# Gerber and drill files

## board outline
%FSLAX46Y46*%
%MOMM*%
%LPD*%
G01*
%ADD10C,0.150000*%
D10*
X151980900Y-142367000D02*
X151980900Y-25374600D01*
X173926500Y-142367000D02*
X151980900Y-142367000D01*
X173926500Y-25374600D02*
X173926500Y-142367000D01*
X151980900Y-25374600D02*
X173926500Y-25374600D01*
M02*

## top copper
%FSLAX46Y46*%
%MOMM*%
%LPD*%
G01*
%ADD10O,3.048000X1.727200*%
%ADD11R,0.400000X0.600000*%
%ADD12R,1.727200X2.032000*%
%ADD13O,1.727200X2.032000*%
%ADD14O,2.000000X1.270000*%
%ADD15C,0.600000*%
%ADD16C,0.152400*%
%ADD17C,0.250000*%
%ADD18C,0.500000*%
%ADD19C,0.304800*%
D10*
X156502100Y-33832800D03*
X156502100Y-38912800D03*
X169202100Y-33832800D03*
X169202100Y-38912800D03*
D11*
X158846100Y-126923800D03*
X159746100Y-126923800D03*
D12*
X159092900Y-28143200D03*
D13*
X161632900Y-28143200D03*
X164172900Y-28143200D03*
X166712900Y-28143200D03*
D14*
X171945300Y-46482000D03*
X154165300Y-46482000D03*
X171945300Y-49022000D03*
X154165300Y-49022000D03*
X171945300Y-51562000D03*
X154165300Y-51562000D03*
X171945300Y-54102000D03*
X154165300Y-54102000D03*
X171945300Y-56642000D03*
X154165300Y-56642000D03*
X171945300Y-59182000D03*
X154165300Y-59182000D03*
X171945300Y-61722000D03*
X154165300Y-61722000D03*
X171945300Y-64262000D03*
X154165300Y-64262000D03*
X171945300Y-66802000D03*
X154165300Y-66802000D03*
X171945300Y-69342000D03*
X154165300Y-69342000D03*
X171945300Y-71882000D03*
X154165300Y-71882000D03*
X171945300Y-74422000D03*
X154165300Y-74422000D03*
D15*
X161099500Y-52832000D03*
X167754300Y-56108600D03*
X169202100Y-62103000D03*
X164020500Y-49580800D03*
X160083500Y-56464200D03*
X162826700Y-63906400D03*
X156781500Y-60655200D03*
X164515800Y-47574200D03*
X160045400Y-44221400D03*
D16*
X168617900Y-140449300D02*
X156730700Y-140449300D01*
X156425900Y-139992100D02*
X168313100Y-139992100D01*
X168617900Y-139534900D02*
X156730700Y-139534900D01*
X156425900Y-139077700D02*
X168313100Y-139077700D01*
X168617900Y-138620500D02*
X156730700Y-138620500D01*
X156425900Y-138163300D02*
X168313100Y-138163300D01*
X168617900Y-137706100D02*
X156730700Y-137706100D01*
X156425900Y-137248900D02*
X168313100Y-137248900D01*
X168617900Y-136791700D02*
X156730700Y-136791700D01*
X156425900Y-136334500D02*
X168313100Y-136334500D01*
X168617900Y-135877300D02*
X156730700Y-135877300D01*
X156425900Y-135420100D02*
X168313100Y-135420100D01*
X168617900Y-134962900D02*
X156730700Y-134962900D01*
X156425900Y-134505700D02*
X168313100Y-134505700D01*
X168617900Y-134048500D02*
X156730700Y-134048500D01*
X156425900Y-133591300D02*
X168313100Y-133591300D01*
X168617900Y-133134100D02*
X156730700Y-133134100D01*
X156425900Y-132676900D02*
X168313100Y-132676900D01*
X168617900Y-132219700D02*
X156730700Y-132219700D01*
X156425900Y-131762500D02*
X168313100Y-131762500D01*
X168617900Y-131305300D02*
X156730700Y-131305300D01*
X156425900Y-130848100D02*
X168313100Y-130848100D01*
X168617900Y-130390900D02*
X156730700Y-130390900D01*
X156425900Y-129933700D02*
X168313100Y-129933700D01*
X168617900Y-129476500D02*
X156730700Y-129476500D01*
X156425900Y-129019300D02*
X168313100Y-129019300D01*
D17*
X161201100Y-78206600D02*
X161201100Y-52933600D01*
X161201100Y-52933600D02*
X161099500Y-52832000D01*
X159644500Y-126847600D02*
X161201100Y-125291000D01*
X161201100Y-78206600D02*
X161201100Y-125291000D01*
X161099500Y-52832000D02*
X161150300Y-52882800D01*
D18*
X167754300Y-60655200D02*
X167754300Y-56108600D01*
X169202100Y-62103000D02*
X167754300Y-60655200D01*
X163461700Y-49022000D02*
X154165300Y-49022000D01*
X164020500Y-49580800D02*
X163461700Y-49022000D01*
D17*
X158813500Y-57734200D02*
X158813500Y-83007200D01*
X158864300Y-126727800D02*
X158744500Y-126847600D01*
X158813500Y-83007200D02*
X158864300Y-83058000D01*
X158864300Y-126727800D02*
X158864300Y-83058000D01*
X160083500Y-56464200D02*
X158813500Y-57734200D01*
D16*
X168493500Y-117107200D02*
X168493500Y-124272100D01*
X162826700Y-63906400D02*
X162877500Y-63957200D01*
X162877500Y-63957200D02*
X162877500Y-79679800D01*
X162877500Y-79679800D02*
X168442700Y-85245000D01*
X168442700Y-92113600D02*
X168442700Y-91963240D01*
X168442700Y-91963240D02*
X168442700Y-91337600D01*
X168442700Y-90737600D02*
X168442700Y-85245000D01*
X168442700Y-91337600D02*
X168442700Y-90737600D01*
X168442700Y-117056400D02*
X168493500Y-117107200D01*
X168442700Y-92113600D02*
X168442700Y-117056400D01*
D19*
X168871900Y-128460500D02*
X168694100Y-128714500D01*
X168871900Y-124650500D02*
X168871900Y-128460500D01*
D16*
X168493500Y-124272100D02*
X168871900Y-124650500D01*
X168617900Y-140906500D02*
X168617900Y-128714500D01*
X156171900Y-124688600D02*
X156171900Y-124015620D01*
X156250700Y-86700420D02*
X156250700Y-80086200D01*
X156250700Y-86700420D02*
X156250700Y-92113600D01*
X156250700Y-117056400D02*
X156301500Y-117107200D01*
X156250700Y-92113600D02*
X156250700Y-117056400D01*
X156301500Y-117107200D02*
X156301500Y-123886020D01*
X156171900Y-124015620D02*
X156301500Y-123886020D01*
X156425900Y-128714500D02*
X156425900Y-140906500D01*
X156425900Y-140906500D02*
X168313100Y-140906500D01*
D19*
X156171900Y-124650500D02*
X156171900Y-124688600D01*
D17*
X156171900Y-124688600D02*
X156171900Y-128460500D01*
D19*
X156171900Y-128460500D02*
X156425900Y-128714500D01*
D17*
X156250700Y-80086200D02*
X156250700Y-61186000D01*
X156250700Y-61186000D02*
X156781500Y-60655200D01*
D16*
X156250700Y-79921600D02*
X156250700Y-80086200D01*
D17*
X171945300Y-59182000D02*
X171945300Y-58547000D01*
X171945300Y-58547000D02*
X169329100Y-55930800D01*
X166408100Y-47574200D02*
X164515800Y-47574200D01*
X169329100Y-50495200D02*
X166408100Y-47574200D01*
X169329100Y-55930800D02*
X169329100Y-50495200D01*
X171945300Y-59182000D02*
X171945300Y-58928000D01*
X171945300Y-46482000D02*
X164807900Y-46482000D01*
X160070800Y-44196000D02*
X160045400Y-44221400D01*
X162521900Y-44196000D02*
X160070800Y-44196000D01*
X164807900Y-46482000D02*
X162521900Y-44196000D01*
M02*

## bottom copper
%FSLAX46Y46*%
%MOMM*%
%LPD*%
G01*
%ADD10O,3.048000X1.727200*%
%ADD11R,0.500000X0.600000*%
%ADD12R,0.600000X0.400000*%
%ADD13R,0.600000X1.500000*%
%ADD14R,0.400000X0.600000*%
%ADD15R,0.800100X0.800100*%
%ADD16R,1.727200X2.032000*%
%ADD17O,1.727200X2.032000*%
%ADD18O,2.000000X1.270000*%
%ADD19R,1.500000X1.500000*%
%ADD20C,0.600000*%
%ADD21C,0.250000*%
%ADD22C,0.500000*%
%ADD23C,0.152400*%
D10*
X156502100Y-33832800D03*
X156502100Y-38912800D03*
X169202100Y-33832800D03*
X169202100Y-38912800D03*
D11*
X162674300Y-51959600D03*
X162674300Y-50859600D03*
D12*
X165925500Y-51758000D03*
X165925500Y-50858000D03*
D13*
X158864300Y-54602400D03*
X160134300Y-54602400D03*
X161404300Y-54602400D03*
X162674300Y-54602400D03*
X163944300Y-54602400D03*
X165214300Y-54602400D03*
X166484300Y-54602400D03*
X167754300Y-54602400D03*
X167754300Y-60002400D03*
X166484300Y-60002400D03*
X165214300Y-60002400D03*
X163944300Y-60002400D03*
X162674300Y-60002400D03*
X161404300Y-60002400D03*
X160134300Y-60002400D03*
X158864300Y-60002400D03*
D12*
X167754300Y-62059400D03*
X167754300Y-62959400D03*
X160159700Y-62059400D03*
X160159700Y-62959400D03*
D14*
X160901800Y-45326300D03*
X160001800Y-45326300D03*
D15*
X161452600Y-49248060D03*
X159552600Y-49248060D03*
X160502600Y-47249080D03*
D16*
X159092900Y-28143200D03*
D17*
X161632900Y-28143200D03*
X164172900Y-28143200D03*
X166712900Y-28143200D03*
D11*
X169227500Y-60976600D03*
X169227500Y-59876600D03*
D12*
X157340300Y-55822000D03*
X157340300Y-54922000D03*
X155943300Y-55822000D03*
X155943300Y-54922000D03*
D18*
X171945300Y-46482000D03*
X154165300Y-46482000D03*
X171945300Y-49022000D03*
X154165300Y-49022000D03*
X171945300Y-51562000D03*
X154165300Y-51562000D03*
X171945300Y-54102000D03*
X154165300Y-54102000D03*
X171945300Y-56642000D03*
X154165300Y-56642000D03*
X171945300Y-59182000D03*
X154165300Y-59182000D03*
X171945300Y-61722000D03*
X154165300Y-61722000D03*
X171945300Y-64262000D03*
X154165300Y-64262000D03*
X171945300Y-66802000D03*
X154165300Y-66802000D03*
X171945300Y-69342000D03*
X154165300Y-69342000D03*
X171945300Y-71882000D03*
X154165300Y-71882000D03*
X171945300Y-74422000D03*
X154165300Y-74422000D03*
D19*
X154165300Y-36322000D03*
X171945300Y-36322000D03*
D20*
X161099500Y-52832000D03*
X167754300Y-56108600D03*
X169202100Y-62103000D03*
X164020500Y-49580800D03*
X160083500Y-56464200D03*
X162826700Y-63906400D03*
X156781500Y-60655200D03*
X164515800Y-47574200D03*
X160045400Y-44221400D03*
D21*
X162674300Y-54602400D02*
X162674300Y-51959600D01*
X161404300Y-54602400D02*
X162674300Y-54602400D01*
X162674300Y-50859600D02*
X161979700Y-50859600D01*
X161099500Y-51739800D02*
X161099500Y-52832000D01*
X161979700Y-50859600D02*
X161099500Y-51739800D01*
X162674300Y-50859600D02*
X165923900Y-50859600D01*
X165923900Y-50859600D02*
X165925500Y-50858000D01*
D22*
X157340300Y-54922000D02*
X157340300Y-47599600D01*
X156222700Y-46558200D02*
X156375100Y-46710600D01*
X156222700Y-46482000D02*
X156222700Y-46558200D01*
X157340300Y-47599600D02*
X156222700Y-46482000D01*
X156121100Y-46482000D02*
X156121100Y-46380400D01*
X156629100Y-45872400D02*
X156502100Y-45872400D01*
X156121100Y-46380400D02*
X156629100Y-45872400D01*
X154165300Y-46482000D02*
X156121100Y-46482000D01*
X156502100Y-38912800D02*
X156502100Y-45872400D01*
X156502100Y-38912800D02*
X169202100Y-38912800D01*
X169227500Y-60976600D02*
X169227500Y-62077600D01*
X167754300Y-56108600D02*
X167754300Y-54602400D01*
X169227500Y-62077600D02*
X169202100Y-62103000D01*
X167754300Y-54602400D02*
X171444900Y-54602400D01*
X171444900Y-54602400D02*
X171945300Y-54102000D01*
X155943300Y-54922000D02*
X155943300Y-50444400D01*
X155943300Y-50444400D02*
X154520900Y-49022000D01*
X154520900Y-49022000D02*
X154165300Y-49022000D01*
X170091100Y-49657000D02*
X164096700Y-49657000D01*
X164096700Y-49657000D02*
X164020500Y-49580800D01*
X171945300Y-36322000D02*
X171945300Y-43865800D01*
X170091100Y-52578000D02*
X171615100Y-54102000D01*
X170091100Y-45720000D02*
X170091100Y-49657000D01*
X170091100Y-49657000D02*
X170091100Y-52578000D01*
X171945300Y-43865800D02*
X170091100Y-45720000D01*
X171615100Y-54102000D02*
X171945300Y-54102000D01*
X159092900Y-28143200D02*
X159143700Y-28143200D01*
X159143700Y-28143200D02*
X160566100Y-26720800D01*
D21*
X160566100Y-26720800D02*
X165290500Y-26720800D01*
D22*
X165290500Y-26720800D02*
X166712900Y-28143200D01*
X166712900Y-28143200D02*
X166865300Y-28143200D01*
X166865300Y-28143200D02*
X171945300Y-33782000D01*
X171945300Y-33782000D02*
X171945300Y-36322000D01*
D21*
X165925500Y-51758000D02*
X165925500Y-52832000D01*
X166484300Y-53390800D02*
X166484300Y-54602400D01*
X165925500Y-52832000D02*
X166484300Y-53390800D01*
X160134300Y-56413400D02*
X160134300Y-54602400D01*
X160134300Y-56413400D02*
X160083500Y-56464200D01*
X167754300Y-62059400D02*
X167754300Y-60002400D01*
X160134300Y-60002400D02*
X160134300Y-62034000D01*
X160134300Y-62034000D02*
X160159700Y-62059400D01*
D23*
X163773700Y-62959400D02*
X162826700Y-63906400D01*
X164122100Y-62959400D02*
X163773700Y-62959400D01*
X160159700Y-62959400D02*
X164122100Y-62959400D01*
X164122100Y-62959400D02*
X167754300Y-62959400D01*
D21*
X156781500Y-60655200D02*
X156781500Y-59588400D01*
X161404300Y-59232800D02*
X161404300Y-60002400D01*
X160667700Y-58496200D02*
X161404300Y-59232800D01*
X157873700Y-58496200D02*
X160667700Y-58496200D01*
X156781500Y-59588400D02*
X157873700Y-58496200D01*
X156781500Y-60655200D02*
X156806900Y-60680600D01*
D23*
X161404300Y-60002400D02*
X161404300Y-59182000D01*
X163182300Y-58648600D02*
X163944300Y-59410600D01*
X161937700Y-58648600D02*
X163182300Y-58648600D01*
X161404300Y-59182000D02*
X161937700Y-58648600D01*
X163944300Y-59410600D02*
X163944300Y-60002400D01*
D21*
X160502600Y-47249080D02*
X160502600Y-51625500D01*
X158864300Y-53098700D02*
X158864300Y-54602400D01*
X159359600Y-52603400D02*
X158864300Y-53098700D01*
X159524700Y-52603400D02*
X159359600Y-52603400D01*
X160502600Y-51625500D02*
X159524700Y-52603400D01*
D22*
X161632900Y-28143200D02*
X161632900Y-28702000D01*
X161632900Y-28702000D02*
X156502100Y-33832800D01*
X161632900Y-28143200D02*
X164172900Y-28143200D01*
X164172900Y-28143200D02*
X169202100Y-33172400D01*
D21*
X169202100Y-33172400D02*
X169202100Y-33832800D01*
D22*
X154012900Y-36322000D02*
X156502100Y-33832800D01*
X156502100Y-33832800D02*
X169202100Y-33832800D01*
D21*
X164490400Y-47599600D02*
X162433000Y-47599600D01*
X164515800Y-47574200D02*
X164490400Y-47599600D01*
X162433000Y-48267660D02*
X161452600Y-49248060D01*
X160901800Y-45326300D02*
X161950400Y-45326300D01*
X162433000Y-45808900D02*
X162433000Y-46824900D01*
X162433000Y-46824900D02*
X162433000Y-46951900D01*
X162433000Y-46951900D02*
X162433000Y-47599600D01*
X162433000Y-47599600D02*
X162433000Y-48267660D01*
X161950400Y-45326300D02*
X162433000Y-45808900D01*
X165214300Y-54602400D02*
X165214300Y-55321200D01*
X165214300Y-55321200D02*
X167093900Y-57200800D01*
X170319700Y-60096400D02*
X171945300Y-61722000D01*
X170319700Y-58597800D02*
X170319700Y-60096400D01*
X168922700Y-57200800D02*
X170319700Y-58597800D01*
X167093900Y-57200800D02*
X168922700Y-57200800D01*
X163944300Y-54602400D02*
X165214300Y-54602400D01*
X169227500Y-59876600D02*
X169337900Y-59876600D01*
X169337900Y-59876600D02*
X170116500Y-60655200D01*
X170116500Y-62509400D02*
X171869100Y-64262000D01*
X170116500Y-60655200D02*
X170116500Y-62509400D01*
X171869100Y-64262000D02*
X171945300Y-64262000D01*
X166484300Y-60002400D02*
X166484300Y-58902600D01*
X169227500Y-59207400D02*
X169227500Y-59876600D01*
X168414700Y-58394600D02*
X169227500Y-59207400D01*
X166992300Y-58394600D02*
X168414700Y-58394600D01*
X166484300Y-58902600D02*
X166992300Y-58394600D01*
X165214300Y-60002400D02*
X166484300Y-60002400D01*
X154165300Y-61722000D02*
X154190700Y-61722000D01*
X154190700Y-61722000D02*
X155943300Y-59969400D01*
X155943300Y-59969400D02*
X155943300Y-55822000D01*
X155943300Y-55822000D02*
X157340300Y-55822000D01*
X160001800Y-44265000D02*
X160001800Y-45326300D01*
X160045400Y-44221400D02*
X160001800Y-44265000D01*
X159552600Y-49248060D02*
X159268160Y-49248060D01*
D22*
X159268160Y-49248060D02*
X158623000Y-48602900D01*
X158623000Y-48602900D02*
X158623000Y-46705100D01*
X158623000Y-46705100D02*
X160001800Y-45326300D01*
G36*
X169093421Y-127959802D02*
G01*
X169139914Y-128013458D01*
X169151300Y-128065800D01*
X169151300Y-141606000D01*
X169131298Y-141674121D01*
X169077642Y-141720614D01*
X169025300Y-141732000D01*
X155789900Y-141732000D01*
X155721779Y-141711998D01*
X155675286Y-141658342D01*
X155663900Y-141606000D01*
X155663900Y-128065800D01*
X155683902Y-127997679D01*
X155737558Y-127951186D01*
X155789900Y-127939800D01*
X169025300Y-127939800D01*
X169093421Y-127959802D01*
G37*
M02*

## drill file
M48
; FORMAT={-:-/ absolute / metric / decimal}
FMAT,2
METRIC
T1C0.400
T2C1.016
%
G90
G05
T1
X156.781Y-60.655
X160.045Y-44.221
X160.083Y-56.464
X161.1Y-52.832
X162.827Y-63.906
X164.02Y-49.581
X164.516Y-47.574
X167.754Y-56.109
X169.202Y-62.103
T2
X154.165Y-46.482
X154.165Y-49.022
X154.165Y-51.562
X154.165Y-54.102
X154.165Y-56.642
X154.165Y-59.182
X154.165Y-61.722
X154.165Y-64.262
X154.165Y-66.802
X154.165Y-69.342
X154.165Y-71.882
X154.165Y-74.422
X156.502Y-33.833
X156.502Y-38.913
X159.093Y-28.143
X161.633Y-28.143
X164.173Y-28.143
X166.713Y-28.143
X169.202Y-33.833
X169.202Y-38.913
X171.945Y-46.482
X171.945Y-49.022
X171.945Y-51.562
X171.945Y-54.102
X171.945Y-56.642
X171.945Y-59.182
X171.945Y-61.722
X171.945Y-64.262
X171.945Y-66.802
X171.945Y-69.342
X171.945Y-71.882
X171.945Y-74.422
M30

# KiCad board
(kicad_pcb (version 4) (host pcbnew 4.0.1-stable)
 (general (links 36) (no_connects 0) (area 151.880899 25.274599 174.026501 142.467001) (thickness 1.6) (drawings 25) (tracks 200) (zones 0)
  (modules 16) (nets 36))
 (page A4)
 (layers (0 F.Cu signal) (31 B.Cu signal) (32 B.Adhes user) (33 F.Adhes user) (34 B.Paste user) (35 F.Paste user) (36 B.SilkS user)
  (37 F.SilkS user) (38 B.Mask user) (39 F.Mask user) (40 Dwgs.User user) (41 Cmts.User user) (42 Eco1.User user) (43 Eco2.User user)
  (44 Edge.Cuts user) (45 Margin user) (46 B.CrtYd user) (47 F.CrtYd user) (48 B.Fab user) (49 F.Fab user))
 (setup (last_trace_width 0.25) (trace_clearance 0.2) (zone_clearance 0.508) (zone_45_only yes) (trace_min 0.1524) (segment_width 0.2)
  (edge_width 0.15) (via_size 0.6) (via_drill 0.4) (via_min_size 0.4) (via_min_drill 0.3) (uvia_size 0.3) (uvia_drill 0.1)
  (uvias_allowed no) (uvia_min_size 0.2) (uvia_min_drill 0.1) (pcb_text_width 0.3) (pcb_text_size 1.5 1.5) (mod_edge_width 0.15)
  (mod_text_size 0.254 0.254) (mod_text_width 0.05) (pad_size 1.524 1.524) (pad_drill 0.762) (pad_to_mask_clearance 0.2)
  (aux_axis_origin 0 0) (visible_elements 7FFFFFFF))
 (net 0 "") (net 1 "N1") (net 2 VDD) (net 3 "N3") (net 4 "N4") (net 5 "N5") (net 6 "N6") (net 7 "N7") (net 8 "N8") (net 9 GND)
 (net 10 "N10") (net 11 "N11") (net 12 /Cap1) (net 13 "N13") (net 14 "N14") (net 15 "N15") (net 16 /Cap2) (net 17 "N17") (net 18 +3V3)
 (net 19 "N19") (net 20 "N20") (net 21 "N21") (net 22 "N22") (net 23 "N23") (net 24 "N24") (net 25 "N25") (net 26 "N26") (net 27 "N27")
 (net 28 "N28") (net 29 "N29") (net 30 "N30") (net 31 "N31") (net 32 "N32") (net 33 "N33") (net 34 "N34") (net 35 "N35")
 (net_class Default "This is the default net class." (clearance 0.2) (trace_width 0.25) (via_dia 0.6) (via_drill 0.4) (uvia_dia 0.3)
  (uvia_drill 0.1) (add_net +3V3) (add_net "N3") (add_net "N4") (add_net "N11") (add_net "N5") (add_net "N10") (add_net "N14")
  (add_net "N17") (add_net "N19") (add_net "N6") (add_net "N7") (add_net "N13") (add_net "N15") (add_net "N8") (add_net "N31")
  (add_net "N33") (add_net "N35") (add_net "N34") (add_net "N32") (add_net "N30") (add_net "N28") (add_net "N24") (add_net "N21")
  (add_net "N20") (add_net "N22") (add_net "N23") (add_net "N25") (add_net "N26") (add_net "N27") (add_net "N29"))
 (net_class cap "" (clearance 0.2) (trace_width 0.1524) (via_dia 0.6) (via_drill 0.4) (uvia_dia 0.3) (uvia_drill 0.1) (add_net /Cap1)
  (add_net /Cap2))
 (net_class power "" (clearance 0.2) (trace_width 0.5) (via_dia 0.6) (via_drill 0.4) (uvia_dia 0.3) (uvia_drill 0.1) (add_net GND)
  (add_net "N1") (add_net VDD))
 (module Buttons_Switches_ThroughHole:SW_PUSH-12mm (layer B.Cu) (at 162.8521 36.3728 180)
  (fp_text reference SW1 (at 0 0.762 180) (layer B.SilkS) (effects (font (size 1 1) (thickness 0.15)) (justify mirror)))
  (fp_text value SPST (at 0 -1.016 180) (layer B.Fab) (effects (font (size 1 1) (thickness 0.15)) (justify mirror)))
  (pad 1 thru_hole oval (at 6.35 2.54 180) (size 3.048 1.7272) (drill 1.016) (layers *.Cu *.Mask B.SilkS) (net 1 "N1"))
  (pad 2 thru_hole oval (at 6.35 -2.54 180) (size 3.048 1.7272) (drill 1.016) (layers *.Cu *.Mask B.SilkS) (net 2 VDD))
  (pad 1 thru_hole oval (at -6.35 2.54 180) (size 3.048 1.7272) (drill 1.016) (layers *.Cu *.Mask B.SilkS) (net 1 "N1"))
  (pad 2 thru_hole oval (at -6.35 -2.54 180) (size 3.048 1.7272) (drill 1.016) (layers *.Cu *.Mask B.SilkS) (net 2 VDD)))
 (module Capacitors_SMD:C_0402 (layer B.Cu) (at 162.6743 51.4096 90)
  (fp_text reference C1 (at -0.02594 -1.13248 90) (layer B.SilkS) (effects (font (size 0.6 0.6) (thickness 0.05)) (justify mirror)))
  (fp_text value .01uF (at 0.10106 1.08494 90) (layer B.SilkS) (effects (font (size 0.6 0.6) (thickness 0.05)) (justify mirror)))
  (pad 1 smd rect (at -0.55 0 90) (size 0.6 0.5) (layers B.Cu B.Paste B.Mask) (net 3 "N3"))
  (pad 2 smd rect (at 0.55 0 90) (size 0.6 0.5) (layers B.Cu B.Paste B.Mask) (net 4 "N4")))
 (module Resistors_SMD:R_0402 (layer B.Cu) (at 165.9255 51.308 90)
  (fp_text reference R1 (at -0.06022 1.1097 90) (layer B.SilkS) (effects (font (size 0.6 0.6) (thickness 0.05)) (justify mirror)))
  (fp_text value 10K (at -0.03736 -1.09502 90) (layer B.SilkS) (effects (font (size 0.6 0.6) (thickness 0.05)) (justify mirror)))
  (pad 1 smd rect (at -0.45 0 90) (size 0.4 0.6) (layers B.Cu B.Paste B.Mask) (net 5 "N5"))
  (pad 2 smd rect (at 0.45 0 90) (size 0.4 0.6) (layers B.Cu B.Paste B.Mask) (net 4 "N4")))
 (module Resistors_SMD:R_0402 (layer F.Cu) (at 159.2961 126.9238)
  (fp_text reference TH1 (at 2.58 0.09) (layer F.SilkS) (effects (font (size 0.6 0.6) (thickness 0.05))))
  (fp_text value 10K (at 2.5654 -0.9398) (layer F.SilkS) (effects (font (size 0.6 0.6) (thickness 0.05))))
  (pad 1 smd rect (at -0.45 0) (size 0.4 0.6) (layers F.Cu F.Paste F.Mask) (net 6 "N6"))
  (pad 2 smd rect (at 0.45 0) (size 0.4 0.6) (layers F.Cu F.Paste F.Mask) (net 4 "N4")))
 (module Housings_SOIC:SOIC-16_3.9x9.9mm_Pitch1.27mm (layer B.Cu) (at 163.3093 57.3024 270)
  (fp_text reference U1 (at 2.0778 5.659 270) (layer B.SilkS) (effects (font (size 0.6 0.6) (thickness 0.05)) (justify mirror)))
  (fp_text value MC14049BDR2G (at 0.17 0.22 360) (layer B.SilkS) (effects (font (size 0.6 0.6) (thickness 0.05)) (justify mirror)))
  (pad 1 smd rect (at -2.7 4.445 270) (size 1.5 0.6) (layers B.Cu B.Paste B.Mask) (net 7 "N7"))
  (pad 2 smd rect (at -2.7 3.175 270) (size 1.5 0.6) (layers B.Cu B.Paste B.Mask) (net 6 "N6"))
  (pad 3 smd rect (at -2.7 1.905 270) (size 1.5 0.6) (layers B.Cu B.Paste B.Mask) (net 3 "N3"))
  (pad 4 smd rect (at -2.7 0.635 270) (size 1.5 0.6) (layers B.Cu B.Paste B.Mask) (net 3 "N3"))
  (pad 5 smd rect (at -2.7 -0.635 270) (size 1.5 0.6) (layers B.Cu B.Paste B.Mask) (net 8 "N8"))
  (pad 6 smd rect (at -2.7 -1.905 270) (size 1.5 0.6) (layers B.Cu B.Paste B.Mask) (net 8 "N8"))
  (pad 7 smd rect (at -2.7 -3.175 270) (size 1.5 0.6) (layers B.Cu B.Paste B.Mask) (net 5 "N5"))
  (pad 8 smd rect (at -2.7 -4.445 270) (size 1.5 0.6) (layers B.Cu B.Paste B.Mask) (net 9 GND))
  (pad 9 smd rect (at 2.7 -4.445 270) (size 1.5 0.6) (layers B.Cu B.Paste B.Mask) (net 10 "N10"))
  (pad 10 smd rect (at 2.7 -3.175 270) (size 1.5 0.6) (layers B.Cu B.Paste B.Mask) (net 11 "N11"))
  (pad 11 smd rect (at 2.7 -1.905 270) (size 1.5 0.6) (layers B.Cu B.Paste B.Mask) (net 11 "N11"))
  (pad 12 smd rect (at 2.7 -0.635 270) (size 1.5 0.6) (layers B.Cu B.Paste B.Mask) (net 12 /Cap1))
  (pad 13 smd rect (at 2.7 0.635 270) (size 1.5 0.6) (layers B.Cu B.Paste B.Mask) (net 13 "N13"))
  (pad 14 smd rect (at 2.7 1.905 270) (size 1.5 0.6) (layers B.Cu B.Paste B.Mask) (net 12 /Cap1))
  (pad 15 smd rect (at 2.7 3.175 270) (size 1.5 0.6) (layers B.Cu B.Paste B.Mask) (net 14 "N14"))
  (pad 16 smd rect (at 2.7 4.445 270) (size 1.5 0.6) (layers B.Cu B.Paste B.Mask) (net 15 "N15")))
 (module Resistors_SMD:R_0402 (layer B.Cu) (at 167.7543 62.5094 270)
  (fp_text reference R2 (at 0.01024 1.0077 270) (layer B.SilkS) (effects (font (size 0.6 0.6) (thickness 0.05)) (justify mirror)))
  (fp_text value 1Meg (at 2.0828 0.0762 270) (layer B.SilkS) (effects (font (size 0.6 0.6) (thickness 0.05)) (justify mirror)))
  (pad 1 smd rect (at -0.45 0 270) (size 0.4 0.6) (layers B.Cu B.Paste B.Mask) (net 10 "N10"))
  (pad 2 smd rect (at 0.45 0 270) (size 0.4 0.6) (layers B.Cu B.Paste B.Mask) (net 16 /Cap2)))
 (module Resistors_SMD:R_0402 (layer B.Cu) (at 160.1597 62.5094 270)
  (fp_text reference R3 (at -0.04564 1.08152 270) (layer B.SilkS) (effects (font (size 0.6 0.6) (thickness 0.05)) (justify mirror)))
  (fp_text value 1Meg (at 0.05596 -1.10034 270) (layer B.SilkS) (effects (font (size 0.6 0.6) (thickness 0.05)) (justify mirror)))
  (pad 1 smd rect (at -0.45 0 270) (size 0.4 0.6) (layers B.Cu B.Paste B.Mask) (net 14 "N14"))
  (pad 2 smd rect (at 0.45 0 270) (size 0.4 0.6) (layers B.Cu B.Paste B.Mask) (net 16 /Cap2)))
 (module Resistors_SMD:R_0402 (layer B.Cu) (at 160.4518 45.3263 180)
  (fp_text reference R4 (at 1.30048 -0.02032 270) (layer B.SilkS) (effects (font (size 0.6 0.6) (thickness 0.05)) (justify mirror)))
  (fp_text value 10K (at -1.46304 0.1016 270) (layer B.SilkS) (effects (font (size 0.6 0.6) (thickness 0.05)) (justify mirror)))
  (pad 1 smd rect (at -0.45 0 180) (size 0.4 0.6) (layers B.Cu B.Paste B.Mask) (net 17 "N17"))
  (pad 2 smd rect (at 0.45 0 180) (size 0.4 0.6) (layers B.Cu B.Paste B.Mask) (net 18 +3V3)))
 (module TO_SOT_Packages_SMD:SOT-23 (layer B.Cu) (at 160.5026 48.2473 180)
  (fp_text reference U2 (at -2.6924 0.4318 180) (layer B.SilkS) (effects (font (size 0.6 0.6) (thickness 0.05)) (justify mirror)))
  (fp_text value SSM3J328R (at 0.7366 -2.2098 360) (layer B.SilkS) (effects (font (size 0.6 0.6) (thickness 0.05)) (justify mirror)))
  (pad 1 smd rect (at -0.95 -1.00076 180) (size 0.8001 0.8001) (layers B.Cu B.Paste B.Mask) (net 17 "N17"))
  (pad 2 smd rect (at 0.95 -1.00076 180) (size 0.8001 0.8001) (layers B.Cu B.Paste B.Mask) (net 18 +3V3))
  (pad 3 smd rect (at 0 0.99822 180) (size 0.8001 0.8001) (layers B.Cu B.Paste B.Mask) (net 7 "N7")))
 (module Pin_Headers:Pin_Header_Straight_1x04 (layer F.Cu) (at 159.0929 28.1432 90)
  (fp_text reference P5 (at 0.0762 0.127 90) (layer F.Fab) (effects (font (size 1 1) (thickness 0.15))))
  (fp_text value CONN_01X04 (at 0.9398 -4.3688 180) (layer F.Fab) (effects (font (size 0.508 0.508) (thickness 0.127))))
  (pad 1 thru_hole rect (at 0 0 90) (size 2.032 1.7272) (drill 1.016) (layers *.Cu *.Mask F.SilkS) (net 9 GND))
  (pad 2 thru_hole oval (at 0 2.54 90) (size 2.032 1.7272) (drill 1.016) (layers *.Cu *.Mask F.SilkS) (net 1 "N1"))
  (pad 3 thru_hole oval (at 0 5.08 90) (size 2.032 1.7272) (drill 1.016) (layers *.Cu *.Mask F.SilkS) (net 1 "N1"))
  (pad 4 thru_hole oval (at 0 7.62 90) (size 2.032 1.7272) (drill 1.016) (layers *.Cu *.Mask F.SilkS) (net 9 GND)))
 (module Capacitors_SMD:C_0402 (layer B.Cu) (at 169.2275 60.4266 90)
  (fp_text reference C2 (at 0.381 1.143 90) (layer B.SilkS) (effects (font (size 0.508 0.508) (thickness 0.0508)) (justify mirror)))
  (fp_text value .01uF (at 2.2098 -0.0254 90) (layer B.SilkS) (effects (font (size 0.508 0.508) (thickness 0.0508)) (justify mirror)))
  (pad 1 smd rect (at -0.55 0 90) (size 0.6 0.5) (layers B.Cu B.Paste B.Mask) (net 9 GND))
  (pad 2 smd rect (at 0.55 0 90) (size 0.6 0.5) (layers B.Cu B.Paste B.Mask) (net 11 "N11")))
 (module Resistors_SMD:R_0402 (layer B.Cu) (at 157.3403 55.372 90)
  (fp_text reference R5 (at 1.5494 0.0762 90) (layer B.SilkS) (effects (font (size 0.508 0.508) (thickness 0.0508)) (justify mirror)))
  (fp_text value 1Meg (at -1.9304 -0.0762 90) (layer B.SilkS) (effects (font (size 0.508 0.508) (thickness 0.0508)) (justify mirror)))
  (pad 1 smd rect (at -0.45 0 90) (size 0.4 0.6) (layers B.Cu B.Paste B.Mask) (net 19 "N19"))
  (pad 2 smd rect (at 0.45 0 90) (size 0.4 0.6) (layers B.Cu B.Paste B.Mask) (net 2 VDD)))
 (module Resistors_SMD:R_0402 (layer B.Cu) (at 155.9433 55.372 90)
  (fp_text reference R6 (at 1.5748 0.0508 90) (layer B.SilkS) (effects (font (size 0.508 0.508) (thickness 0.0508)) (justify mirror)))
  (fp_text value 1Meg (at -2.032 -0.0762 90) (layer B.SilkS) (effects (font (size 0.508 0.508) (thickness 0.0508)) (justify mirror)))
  (pad 1 smd rect (at -0.45 0 90) (size 0.4 0.6) (layers B.Cu B.Paste B.Mask) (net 19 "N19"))
  (pad 2 smd rect (at 0.45 0 90) (size 0.4 0.6) (layers B.Cu B.Paste B.Mask) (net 9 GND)))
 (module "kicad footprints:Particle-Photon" (layer F.Cu) (at 163.0553 60.452 270)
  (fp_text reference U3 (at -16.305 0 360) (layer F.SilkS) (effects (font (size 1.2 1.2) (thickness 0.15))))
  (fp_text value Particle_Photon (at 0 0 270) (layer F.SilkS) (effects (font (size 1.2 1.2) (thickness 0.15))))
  (pad 24 thru_hole oval (at -13.97 -8.89 270) (size 1.27 2) (drill 1.016) (layers *.Cu *.Mask F.SilkS) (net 18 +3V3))
  (pad 1 thru_hole oval (at -13.97 8.89 270) (size 1.27 2) (drill 1.016) (layers *.Cu *.Mask F.SilkS) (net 2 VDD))
  (pad 23 thru_hole oval (at -11.43 -8.89 270) (size 1.27 2) (drill 1.016) (layers *.Cu *.Mask F.SilkS) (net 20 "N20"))
  (pad 2 thru_hole oval (at -11.43 8.89 270) (size 1.27 2) (drill 1.016) (layers *.Cu *.Mask F.SilkS) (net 9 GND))
  (pad 22 thru_hole oval (at -8.89 -8.89 270) (size 1.27 2) (drill 1.016) (layers *.Cu *.Mask F.SilkS) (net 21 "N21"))
  (pad 3 thru_hole oval (at -8.89 8.89 270) (size 1.27 2) (drill 1.016) (layers *.Cu *.Mask F.SilkS) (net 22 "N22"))
  (pad 21 thru_hole oval (at -6.35 -8.89 270) (size 1.27 2) (drill 1.016) (layers *.Cu *.Mask F.SilkS) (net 9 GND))
  (pad 4 thru_hole oval (at -6.35 8.89 270) (size 1.27 2) (drill 1.016) (layers *.Cu *.Mask F.SilkS) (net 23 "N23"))
  (pad 20 thru_hole oval (at -3.81 -8.89 270) (size 1.27 2) (drill 1.016) (layers *.Cu *.Mask F.SilkS) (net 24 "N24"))
  (pad 5 thru_hole oval (at -3.81 8.89 270) (size 1.27 2) (drill 1.016) (layers *.Cu *.Mask F.SilkS) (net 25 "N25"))
  (pad 19 thru_hole oval (at -1.27 -8.89 270) (size 1.27 2) (drill 1.016) (layers *.Cu *.Mask F.SilkS) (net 17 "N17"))
  (pad 6 thru_hole oval (at -1.27 8.89 270) (size 1.27 2) (drill 1.016) (layers *.Cu *.Mask F.SilkS) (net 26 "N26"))
  (pad 18 thru_hole oval (at 1.27 -8.89 270) (size 1.27 2) (drill 1.016) (layers *.Cu *.Mask F.SilkS) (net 8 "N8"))
  (pad 7 thru_hole oval (at 1.27 8.89 270) (size 1.27 2) (drill 1.016) (layers *.Cu *.Mask F.SilkS) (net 19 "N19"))
  (pad 17 thru_hole oval (at 3.81 -8.89 270) (size 1.27 2) (drill 1.016) (layers *.Cu *.Mask F.SilkS) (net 11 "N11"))
  (pad 8 thru_hole oval (at 3.81 8.89 270) (size 1.27 2) (drill 1.016) (layers *.Cu *.Mask F.SilkS) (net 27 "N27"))
  (pad 16 thru_hole oval (at 6.35 -8.89 270) (size 1.27 2) (drill 1.016) (layers *.Cu *.Mask F.SilkS) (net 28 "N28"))
  (pad 9 thru_hole oval (at 6.35 8.89 270) (size 1.27 2) (drill 1.016) (layers *.Cu *.Mask F.SilkS) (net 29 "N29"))
  (pad 15 thru_hole oval (at 8.89 -8.89 270) (size 1.27 2) (drill 1.016) (layers *.Cu *.Mask F.SilkS) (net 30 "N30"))
  (pad 10 thru_hole oval (at 8.89 8.89 270) (size 1.27 2) (drill 1.016) (layers *.Cu *.Mask F.SilkS) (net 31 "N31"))
  (pad 14 thru_hole oval (at 11.43 -8.89 270) (size 1.27 2) (drill 1.016) (layers *.Cu *.Mask F.SilkS) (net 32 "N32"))
  (pad 11 thru_hole oval (at 11.43 8.89 270) (size 1.27 2) (drill 1.016) (layers *.Cu *.Mask F.SilkS) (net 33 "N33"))
  (pad 13 thru_hole oval (at 13.97 -8.89 270) (size 1.27 2) (drill 1.016) (layers *.Cu *.Mask F.SilkS) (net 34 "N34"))
  (pad 12 thru_hole oval (at 13.97 8.89 270) (size 1.27 2) (drill 1.016) (layers *.Cu *.Mask F.SilkS) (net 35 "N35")))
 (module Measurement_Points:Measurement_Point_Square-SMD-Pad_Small (layer B.Cu) (at 154.1653 36.322)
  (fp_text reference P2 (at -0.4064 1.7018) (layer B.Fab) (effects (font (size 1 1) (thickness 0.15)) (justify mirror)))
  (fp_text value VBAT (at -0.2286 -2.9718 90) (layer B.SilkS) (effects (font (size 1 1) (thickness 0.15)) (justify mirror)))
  (pad 1 smd rect (at 0 0) (size 1.5 1.5) (layers B.Cu B.Mask) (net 1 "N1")))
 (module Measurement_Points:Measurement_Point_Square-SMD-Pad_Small (layer B.Cu) (at 171.9453 36.322)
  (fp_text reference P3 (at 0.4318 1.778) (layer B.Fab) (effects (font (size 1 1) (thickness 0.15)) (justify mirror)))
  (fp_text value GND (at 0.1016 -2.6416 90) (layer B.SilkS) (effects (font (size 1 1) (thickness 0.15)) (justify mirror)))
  (pad 1 smd rect (at 0 0) (size 1.5 1.5) (layers B.Cu B.Mask) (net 9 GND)))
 (gr_line (start 151.9809 142.367) (end 151.9809 25.3746) (angle 90) (layer Edge.Cuts) (width 0.15))
 (gr_line (start 173.9265 142.367) (end 151.9809 142.367) (angle 90) (layer Edge.Cuts) (width 0.15))
 (gr_line (start 173.9265 25.3746) (end 173.9265 142.367) (angle 90) (layer Edge.Cuts) (width 0.15))
 (gr_line (start 151.9809 25.3746) (end 173.9265 25.3746) (angle 90) (layer Edge.Cuts) (width 0.15))
 (segment (start 168.6179 140.4493) (end 156.7307 140.4493) (width 0.1524) (layer F.Cu) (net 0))
 (segment (start 156.4259 139.9921) (end 168.3131 139.9921) (width 0.1524) (layer F.Cu) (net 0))
 (segment (start 168.6179 139.5349) (end 156.7307 139.5349) (width 0.1524) (layer F.Cu) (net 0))
 (segment (start 156.4259 139.0777) (end 168.3131 139.0777) (width 0.1524) (layer F.Cu) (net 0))
 (segment (start 168.6179 138.6205) (end 156.7307 138.6205) (width 0.1524) (layer F.Cu) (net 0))
 (segment (start 156.4259 138.1633) (end 168.3131 138.1633) (width 0.1524) (layer F.Cu) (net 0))
 (segment (start 168.6179 137.7061) (end 156.7307 137.7061) (width 0.1524) (layer F.Cu) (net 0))
 (segment (start 156.4259 137.2489) (end 168.3131 137.2489) (width 0.1524) (layer F.Cu) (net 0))
 (segment (start 168.6179 136.7917) (end 156.7307 136.7917) (width 0.1524) (layer F.Cu) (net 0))
 (segment (start 156.4259 136.3345) (end 168.3131 136.3345) (width 0.1524) (layer F.Cu) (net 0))
 (segment (start 168.6179 135.8773) (end 156.7307 135.8773) (width 0.1524) (layer F.Cu) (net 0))
 (segment (start 156.4259 135.4201) (end 168.3131 135.4201) (width 0.1524) (layer F.Cu) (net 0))
 (segment (start 168.6179 134.9629) (end 156.7307 134.9629) (width 0.1524) (layer F.Cu) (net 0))
 (segment (start 156.4259 134.5057) (end 168.3131 134.5057) (width 0.1524) (layer F.Cu) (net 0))
 (segment (start 168.6179 134.0485) (end 156.7307 134.0485) (width 0.1524) (layer F.Cu) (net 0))
 (segment (start 156.4259 133.5913) (end 168.3131 133.5913) (width 0.1524) (layer F.Cu) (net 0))
 (segment (start 168.6179 133.1341) (end 156.7307 133.1341) (width 0.1524) (layer F.Cu) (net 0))
 (segment (start 156.4259 132.6769) (end 168.3131 132.6769) (width 0.1524) (layer F.Cu) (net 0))
 (segment (start 168.6179 132.2197) (end 156.7307 132.2197) (width 0.1524) (layer F.Cu) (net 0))
 (segment (start 156.4259 131.7625) (end 168.3131 131.7625) (width 0.1524) (layer F.Cu) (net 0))
 (segment (start 168.6179 131.3053) (end 156.7307 131.3053) (width 0.1524) (layer F.Cu) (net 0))
 (segment (start 156.4259 130.8481) (end 168.3131 130.8481) (width 0.1524) (layer F.Cu) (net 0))
 (segment (start 168.6179 130.3909) (end 156.7307 130.3909) (width 0.1524) (layer F.Cu) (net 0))
 (segment (start 156.4259 129.9337) (end 168.3131 129.9337) (width 0.1524) (layer F.Cu) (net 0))
 (segment (start 168.6179 129.4765) (end 156.7307 129.4765) (width 0.1524) (layer F.Cu) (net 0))
 (segment (start 156.4259 129.0193) (end 168.3131 129.0193) (width 0.1524) (layer F.Cu) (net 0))
 (segment (start 162.6743 54.6024) (end 162.6743 51.9596) (width 0.25) (layer B.Cu) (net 3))
 (segment (start 161.4043 54.6024) (end 162.6743 54.6024) (width 0.25) (layer B.Cu) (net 3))
 (segment (start 161.2011 78.2066) (end 161.2011 52.9336) (width 0.25) (layer F.Cu) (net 4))
 (segment (start 161.2011 52.9336) (end 161.0995 52.832) (width 0.25) (layer F.Cu) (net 4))
 (segment (start 159.6445 126.8476) (end 161.2011 125.291) (width 0.25) (layer F.Cu) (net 4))
 (segment (start 161.2011 78.2066) (end 161.2011 125.291) (width 0.25) (layer F.Cu) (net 4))
 (segment (start 162.6743 50.8596) (end 161.9797 50.8596) (width 0.25) (layer B.Cu) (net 4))
 (segment (start 161.0995 52.832) (end 161.1503 52.8828) (width 0.25) (layer F.Cu) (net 4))
 (via (at 161.0995 52.832) (size 0.6) (drill 0.4) (layers F.Cu B.Cu) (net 4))
 (segment (start 161.0995 51.7398) (end 161.0995 52.832) (width 0.25) (layer B.Cu) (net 4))
 (segment (start 161.9797 50.8596) (end 161.0995 51.7398) (width 0.25) (layer B.Cu) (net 4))
 (segment (start 162.6743 50.8596) (end 165.9239 50.8596) (width 0.25) (layer B.Cu) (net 4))
 (segment (start 165.9239 50.8596) (end 165.9255 50.858) (width 0.25) (layer B.Cu) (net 4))
 (segment (start 157.3403 54.922) (end 157.3403 47.5996) (width 0.5) (layer B.Cu) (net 2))
 (segment (start 156.2227 46.5582) (end 156.3751 46.7106) (width 0.5) (layer B.Cu) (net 2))
 (segment (start 156.2227 46.482) (end 156.2227 46.5582) (width 0.5) (layer B.Cu) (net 2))
 (segment (start 157.3403 47.5996) (end 156.2227 46.482) (width 0.5) (layer B.Cu) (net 2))
 (segment (start 156.1211 46.482) (end 156.1211 46.3804) (width 0.5) (layer B.Cu) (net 2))
 (segment (start 156.6291 45.8724) (end 156.5021 45.8724) (width 0.5) (layer B.Cu) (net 2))
 (segment (start 156.1211 46.3804) (end 156.6291 45.8724) (width 0.5) (layer B.Cu) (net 2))
 (segment (start 154.1653 46.482) (end 156.1211 46.482) (width 0.5) (layer B.Cu) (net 2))
 (segment (start 156.5021 38.9128) (end 156.5021 45.8724) (width 0.5) (layer B.Cu) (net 2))
 (segment (start 156.5021 38.9128) (end 169.2021 38.9128) (width 0.5) (layer B.Cu) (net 2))
 (segment (start 169.2275 60.9766) (end 169.2275 62.0776) (width 0.5) (layer B.Cu) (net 9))
 (segment (start 167.7543 56.1086) (end 167.7543 54.6024) (width 0.5) (layer B.Cu) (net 9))
 (via (at 167.7543 56.1086) (size 0.6) (drill 0.4) (layers F.Cu B.Cu) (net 9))
 (segment (start 167.7543 60.6552) (end 167.7543 56.1086) (width 0.5) (layer F.Cu) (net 9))
 (segment (start 169.2021 62.103) (end 167.7543 60.6552) (width 0.5) (layer F.Cu) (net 9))
 (via (at 169.2021 62.103) (size 0.6) (drill 0.4) (layers F.Cu B.Cu) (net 9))
 (segment (start 169.2275 62.0776) (end 169.2021 62.103) (width 0.5) (layer B.Cu) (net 9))
 (segment (start 167.7543 54.6024) (end 171.4449 54.6024) (width 0.5) (layer B.Cu) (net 9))
 (segment (start 171.4449 54.6024) (end 171.9453 54.102) (width 0.5) (layer B.Cu) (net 9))
 (segment (start 155.9433 54.922) (end 155.9433 50.4444) (width 0.5) (layer B.Cu) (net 9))
 (segment (start 155.9433 50.4444) (end 154.5209 49.022) (width 0.5) (layer B.Cu) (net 9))
 (segment (start 154.5209 49.022) (end 154.1653 49.022) (width 0.5) (layer B.Cu) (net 9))
 (segment (start 170.0911 49.657) (end 164.0967 49.657) (width 0.5) (layer B.Cu) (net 9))
 (segment (start 163.4617 49.022) (end 154.1653 49.022) (width 0.5) (layer F.Cu) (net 9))
 (segment (start 164.0205 49.5808) (end 163.4617 49.022) (width 0.5) (layer F.Cu) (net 9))
 (via (at 164.0205 49.5808) (size 0.6) (drill 0.4) (layers F.Cu B.Cu) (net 9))
 (segment (start 164.0967 49.657) (end 164.0205 49.5808) (width 0.5) (layer B.Cu) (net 9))
 (segment (start 171.9453 36.322) (end 171.9453 43.8658) (width 0.5) (layer B.Cu) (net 9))
 (segment (start 170.0911 52.578) (end 171.6151 54.102) (width 0.5) (layer B.Cu) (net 9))
 (segment (start 170.0911 45.72) (end 170.0911 49.657) (width 0.5) (layer B.Cu) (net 9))
 (segment (start 170.0911 49.657) (end 170.0911 52.578) (width 0.5) (layer B.Cu) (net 9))
 (segment (start 171.9453 43.8658) (end 170.0911 45.72) (width 0.5) (layer B.Cu) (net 9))
 (segment (start 171.6151 54.102) (end 171.9453 54.102) (width 0.5) (layer B.Cu) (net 9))
 (segment (start 159.0929 28.1432) (end 159.1437 28.1432) (width 0.5) (layer B.Cu) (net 9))
 (segment (start 159.1437 28.1432) (end 160.5661 26.7208) (width 0.5) (layer B.Cu) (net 9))
 (segment (start 160.5661 26.7208) (end 165.2905 26.7208) (width 0.25) (layer B.Cu) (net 9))
 (segment (start 165.2905 26.7208) (end 166.7129 28.1432) (width 0.5) (layer B.Cu) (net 9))
 (segment (start 166.7129 28.1432) (end 166.8653 28.1432) (width 0.5) (layer B.Cu) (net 9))
 (segment (start 166.8653 28.1432) (end 171.9453 33.782) (width 0.5) (layer B.Cu) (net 9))
 (segment (start 171.9453 33.782) (end 171.9453 36.322) (width 0.5) (layer B.Cu) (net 9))
 (segment (start 165.9255 51.758) (end 165.9255 52.832) (width 0.25) (layer B.Cu) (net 5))
 (segment (start 166.4843 53.3908) (end 166.4843 54.6024) (width 0.25) (layer B.Cu) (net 5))
 (segment (start 165.9255 52.832) (end 166.4843 53.3908) (width 0.25) (layer B.Cu) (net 5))
 (segment (start 158.8135 57.7342) (end 158.8135 83.0072) (width 0.25) (layer F.Cu) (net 6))
 (segment (start 158.8643 126.7278) (end 158.7445 126.8476) (width 0.25) (layer F.Cu) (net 6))
 (segment (start 158.8135 83.0072) (end 158.8643 83.058) (width 0.25) (layer F.Cu) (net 6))
 (segment (start 160.1343 56.4134) (end 160.1343 54.6024) (width 0.25) (layer B.Cu) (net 6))
 (segment (start 158.8643 126.7278) (end 158.8643 83.058) (width 0.25) (layer F.Cu) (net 6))
 (segment (start 160.0835 56.4642) (end 158.8135 57.7342) (width 0.25) (layer F.Cu) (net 6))
 (via (at 160.0835 56.4642) (size 0.6) (drill 0.4) (layers F.Cu B.Cu) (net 6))
 (segment (start 160.1343 56.4134) (end 160.0835 56.4642) (width 0.25) (layer B.Cu) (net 6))
 (segment (start 167.7543 62.0594) (end 167.7543 60.0024) (width 0.25) (layer B.Cu) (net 10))
 (segment (start 160.1343 60.0024) (end 160.1343 62.034) (width 0.25) (layer B.Cu) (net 14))
 (segment (start 160.1343 62.034) (end 160.1597 62.0594) (width 0.25) (layer B.Cu) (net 14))
 (segment (start 168.4935 117.1072) (end 168.4935 124.2721) (width 0.1524) (layer F.Cu) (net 16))
 (segment (start 163.7737 62.9594) (end 162.8267 63.9064) (width 0.1524) (layer B.Cu) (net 16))
 (via (at 162.8267 63.9064) (size 0.6) (drill 0.4) (layers F.Cu B.Cu) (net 16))
 (segment (start 162.8267 63.9064) (end 162.8775 63.9572) (width 0.1524) (layer F.Cu) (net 16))
 (segment (start 162.8775 63.9572) (end 162.8775 79.6798) (width 0.1524) (layer F.Cu) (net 16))
 (segment (start 162.8775 79.6798) (end 168.4427 85.245) (width 0.1524) (layer F.Cu) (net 16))
 (segment (start 164.1221 62.9594) (end 163.7737 62.9594) (width 0.1524) (layer B.Cu) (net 16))
 (segment (start 168.4427 92.1136) (end 168.4427 91.96324) (width 0.1524) (layer F.Cu) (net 16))
 (segment (start 168.4427 91.96324) (end 168.4427 91.3376) (width 0.1524) (layer F.Cu) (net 16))
 (segment (start 168.4427 90.7376) (end 168.4427 85.245) (width 0.1524) (layer F.Cu) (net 16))
 (segment (start 168.4427 91.3376) (end 168.4427 90.7376) (width 0.1524) (layer F.Cu) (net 16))
 (segment (start 168.4427 117.0564) (end 168.4935 117.1072) (width 0.1524) (layer F.Cu) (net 16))
 (segment (start 168.4427 92.1136) (end 168.4427 117.0564) (width 0.1524) (layer F.Cu) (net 16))
 (segment (start 168.8719 128.4605) (end 168.6941 128.7145) (width 0.3048) (layer F.Cu) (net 16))
 (segment (start 168.8719 124.6505) (end 168.8719 128.4605) (width 0.3048) (layer F.Cu) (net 16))
 (segment (start 168.4935 124.2721) (end 168.8719 124.6505) (width 0.1524) (layer F.Cu) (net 16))
 (segment (start 168.6179 140.9065) (end 168.6179 128.7145) (width 0.1524) (layer F.Cu) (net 16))
 (segment (start 160.1597 62.9594) (end 164.1221 62.9594) (width 0.1524) (layer B.Cu) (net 16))
 (segment (start 164.1221 62.9594) (end 167.7543 62.9594) (width 0.1524) (layer B.Cu) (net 16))
 (segment (start 156.1719 124.6886) (end 156.1719 124.01562) (width 0.1524) (layer F.Cu) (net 12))
 (segment (start 156.2507 86.70042) (end 156.2507 80.0862) (width 0.1524) (layer F.Cu) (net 12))
 (segment (start 156.2507 86.70042) (end 156.2507 92.1136) (width 0.1524) (layer F.Cu) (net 12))
 (segment (start 156.2507 117.0564) (end 156.3015 117.1072) (width 0.1524) (layer F.Cu) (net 12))
 (segment (start 156.2507 92.1136) (end 156.2507 117.0564) (width 0.1524) (layer F.Cu) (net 12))
 (segment (start 156.3015 117.1072) (end 156.3015 123.88602) (width 0.1524) (layer F.Cu) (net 12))
 (segment (start 156.1719 124.01562) (end 156.3015 123.88602) (width 0.1524) (layer F.Cu) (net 12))
 (segment (start 156.4259 128.7145) (end 156.4259 140.9065) (width 0.1524) (layer F.Cu) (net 12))
 (segment (start 156.4259 140.9065) (end 168.3131 140.9065) (width 0.1524) (layer F.Cu) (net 12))
 (segment (start 156.1719 124.6505) (end 156.1719 124.6886) (width 0.3048) (layer F.Cu) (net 12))
 (segment (start 156.1719 124.6886) (end 156.1719 128.4605) (width 0.25) (layer F.Cu) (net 12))
 (segment (start 156.1719 128.4605) (end 156.4259 128.7145) (width 0.3048) (layer F.Cu) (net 12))
 (segment (start 156.7815 60.6552) (end 156.7815 59.5884) (width 0.25) (layer B.Cu) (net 12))
 (segment (start 161.4043 59.2328) (end 161.4043 60.0024) (width 0.25) (layer B.Cu) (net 12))
 (segment (start 160.6677 58.4962) (end 161.4043 59.2328) (width 0.25) (layer B.Cu) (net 12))
 (segment (start 157.8737 58.4962) (end 160.6677 58.4962) (width 0.25) (layer B.Cu) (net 12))
 (segment (start 156.7815 59.5884) (end 157.8737 58.4962) (width 0.25) (layer B.Cu) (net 12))
 (segment (start 156.2507 80.0862) (end 156.2507 61.186) (width 0.25) (layer F.Cu) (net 12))
 (segment (start 156.7815 60.6552) (end 156.8069 60.6806) (width 0.25) (layer B.Cu) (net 12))
 (via (at 156.7815 60.6552) (size 0.6) (drill 0.4) (layers F.Cu B.Cu) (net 12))
 (segment (start 156.2507 61.186) (end 156.7815 60.6552) (width 0.25) (layer F.Cu) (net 12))
 (segment (start 156.2507 79.9216) (end 156.2507 80.0862) (width 0.1524) (layer F.Cu) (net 12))
 (segment (start 161.4043 60.0024) (end 161.4043 59.182) (width 0.1524) (layer B.Cu) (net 12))
 (segment (start 163.1823 58.6486) (end 163.9443 59.4106) (width 0.1524) (layer B.Cu) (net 12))
 (segment (start 161.9377 58.6486) (end 163.1823 58.6486) (width 0.1524) (layer B.Cu) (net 12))
 (segment (start 161.4043 59.182) (end 161.9377 58.6486) (width 0.1524) (layer B.Cu) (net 12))
 (segment (start 163.9443 59.4106) (end 163.9443 60.0024) (width 0.1524) (layer B.Cu) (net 12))
 (segment (start 160.5026 47.24908) (end 160.5026 51.6255) (width 0.25) (layer B.Cu) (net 7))
 (segment (start 158.8643 53.0987) (end 158.8643 54.6024) (width 0.25) (layer B.Cu) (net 7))
 (segment (start 159.3596 52.6034) (end 158.8643 53.0987) (width 0.25) (layer B.Cu) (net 7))
 (segment (start 159.5247 52.6034) (end 159.3596 52.6034) (width 0.25) (layer B.Cu) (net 7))
 (segment (start 160.5026 51.6255) (end 159.5247 52.6034) (width 0.25) (layer B.Cu) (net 7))
 (segment (start 161.6329 28.1432) (end 161.6329 28.702) (width 0.5) (layer B.Cu) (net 1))
 (segment (start 161.6329 28.702) (end 156.5021 33.8328) (width 0.5) (layer B.Cu) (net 1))
 (segment (start 161.6329 28.1432) (end 164.1729 28.1432) (width 0.5) (layer B.Cu) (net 1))
 (segment (start 164.1729 28.1432) (end 169.2021 33.1724) (width 0.5) (layer B.Cu) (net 1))
 (segment (start 169.2021 33.1724) (end 169.2021 33.8328) (width 0.25) (layer B.Cu) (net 1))
 (segment (start 154.0129 36.322) (end 156.5021 33.8328) (width 0.5) (layer B.Cu) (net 1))
 (segment (start 156.5021 33.8328) (end 169.2021 33.8328) (width 0.5) (layer B.Cu) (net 1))
 (segment (start 171.9453 59.182) (end 171.9453 58.547) (width 0.25) (layer F.Cu) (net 17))
 (segment (start 171.9453 58.547) (end 169.3291 55.9308) (width 0.25) (layer F.Cu) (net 17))
 (segment (start 164.4904 47.5996) (end 162.433 47.5996) (width 0.25) (layer B.Cu) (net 17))
 (segment (start 164.5158 47.5742) (end 164.4904 47.5996) (width 0.25) (layer B.Cu) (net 17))
 (via (at 164.5158 47.5742) (size 0.6) (drill 0.4) (layers F.Cu B.Cu) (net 17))
 (segment (start 166.4081 47.5742) (end 164.5158 47.5742) (width 0.25) (layer F.Cu) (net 17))
 (segment (start 169.3291 50.4952) (end 166.4081 47.5742) (width 0.25) (layer F.Cu) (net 17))
 (segment (start 169.3291 55.9308) (end 169.3291 50.4952) (width 0.25) (layer F.Cu) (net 17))
 (segment (start 171.9453 59.182) (end 171.9453 58.928) (width 0.25) (layer F.Cu) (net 17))
 (segment (start 162.433 48.26766) (end 161.4526 49.24806) (width 0.25) (layer B.Cu) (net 17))
 (segment (start 160.9018 45.3263) (end 161.9504 45.3263) (width 0.25) (layer B.Cu) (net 17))
 (segment (start 162.433 45.8089) (end 162.433 46.8249) (width 0.25) (layer B.Cu) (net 17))
 (segment (start 162.433 46.8249) (end 162.433 46.9519) (width 0.25) (layer B.Cu) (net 17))
 (segment (start 162.433 46.9519) (end 162.433 47.5996) (width 0.25) (layer B.Cu) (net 17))
 (segment (start 162.433 47.5996) (end 162.433 48.26766) (width 0.25) (layer B.Cu) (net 17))
 (segment (start 161.9504 45.3263) (end 162.433 45.8089) (width 0.25) (layer B.Cu) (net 17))
 (segment (start 165.2143 54.6024) (end 165.2143 55.3212) (width 0.25) (layer B.Cu) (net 8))
 (segment (start 165.2143 55.3212) (end 167.0939 57.2008) (width 0.25) (layer B.Cu) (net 8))
 (segment (start 170.3197 60.0964) (end 171.9453 61.722) (width 0.25) (layer B.Cu) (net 8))
 (segment (start 170.3197 58.5978) (end 170.3197 60.0964) (width 0.25) (layer B.Cu) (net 8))
 (segment (start 168.9227 57.2008) (end 170.3197 58.5978) (width 0.25) (layer B.Cu) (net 8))
 (segment (start 167.0939 57.2008) (end 168.9227 57.2008) (width 0.25) (layer B.Cu) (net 8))
 (segment (start 163.9443 54.6024) (end 165.2143 54.6024) (width 0.25) (layer B.Cu) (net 8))
 (segment (start 169.2275 59.8766) (end 169.3379 59.8766) (width 0.25) (layer B.Cu) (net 11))
 (segment (start 169.3379 59.8766) (end 170.1165 60.6552) (width 0.25) (layer B.Cu) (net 11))
 (segment (start 170.1165 62.5094) (end 171.8691 64.262) (width 0.25) (layer B.Cu) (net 11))
 (segment (start 170.1165 60.6552) (end 170.1165 62.5094) (width 0.25) (layer B.Cu) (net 11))
 (segment (start 171.8691 64.262) (end 171.9453 64.262) (width 0.25) (layer B.Cu) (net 11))
 (segment (start 166.4843 60.0024) (end 166.4843 58.9026) (width 0.25) (layer B.Cu) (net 11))
 (segment (start 169.2275 59.2074) (end 169.2275 59.8766) (width 0.25) (layer B.Cu) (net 11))
 (segment (start 168.4147 58.3946) (end 169.2275 59.2074) (width 0.25) (layer B.Cu) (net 11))
 (segment (start 166.9923 58.3946) (end 168.4147 58.3946) (width 0.25) (layer B.Cu) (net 11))
 (segment (start 166.4843 58.9026) (end 166.9923 58.3946) (width 0.25) (layer B.Cu) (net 11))
 (segment (start 165.2143 60.0024) (end 166.4843 60.0024) (width 0.25) (layer B.Cu) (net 11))
 (segment (start 154.1653 61.722) (end 154.1907 61.722) (width 0.25) (layer B.Cu) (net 19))
 (segment (start 154.1907 61.722) (end 155.9433 59.9694) (width 0.25) (layer B.Cu) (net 19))
 (segment (start 155.9433 59.9694) (end 155.9433 55.822) (width 0.25) (layer B.Cu) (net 19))
 (segment (start 155.9433 55.822) (end 157.3403 55.822) (width 0.25) (layer B.Cu) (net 19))
 (segment (start 171.9453 46.482) (end 164.8079 46.482) (width 0.25) (layer F.Cu) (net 18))
 (segment (start 160.0018 44.265) (end 160.0018 45.3263) (width 0.25) (layer B.Cu) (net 18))
 (segment (start 160.0454 44.2214) (end 160.0018 44.265) (width 0.25) (layer B.Cu) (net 18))
 (via (at 160.0454 44.2214) (size 0.6) (drill 0.4) (layers F.Cu B.Cu) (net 18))
 (segment (start 160.0708 44.196) (end 160.0454 44.2214) (width 0.25) (layer F.Cu) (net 18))
 (segment (start 162.5219 44.196) (end 160.0708 44.196) (width 0.25) (layer F.Cu) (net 18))
 (segment (start 164.8079 46.482) (end 162.5219 44.196) (width 0.25) (layer F.Cu) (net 18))
 (segment (start 159.5526 49.24806) (end 159.26816 49.24806) (width 0.25) (layer B.Cu) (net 18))
 (segment (start 159.26816 49.24806) (end 158.623 48.6029) (width 0.5) (layer B.Cu) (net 18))
 (segment (start 158.623 48.6029) (end 158.623 46.7051) (width 0.5) (layer B.Cu) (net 18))
 (segment (start 158.623 46.7051) (end 160.0018 45.3263) (width 0.5) (layer B.Cu) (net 18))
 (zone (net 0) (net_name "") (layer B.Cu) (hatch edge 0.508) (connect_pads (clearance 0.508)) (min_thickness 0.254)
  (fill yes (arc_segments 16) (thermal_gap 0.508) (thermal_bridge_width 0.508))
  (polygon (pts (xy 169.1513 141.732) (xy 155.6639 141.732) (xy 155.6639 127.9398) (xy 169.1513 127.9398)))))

